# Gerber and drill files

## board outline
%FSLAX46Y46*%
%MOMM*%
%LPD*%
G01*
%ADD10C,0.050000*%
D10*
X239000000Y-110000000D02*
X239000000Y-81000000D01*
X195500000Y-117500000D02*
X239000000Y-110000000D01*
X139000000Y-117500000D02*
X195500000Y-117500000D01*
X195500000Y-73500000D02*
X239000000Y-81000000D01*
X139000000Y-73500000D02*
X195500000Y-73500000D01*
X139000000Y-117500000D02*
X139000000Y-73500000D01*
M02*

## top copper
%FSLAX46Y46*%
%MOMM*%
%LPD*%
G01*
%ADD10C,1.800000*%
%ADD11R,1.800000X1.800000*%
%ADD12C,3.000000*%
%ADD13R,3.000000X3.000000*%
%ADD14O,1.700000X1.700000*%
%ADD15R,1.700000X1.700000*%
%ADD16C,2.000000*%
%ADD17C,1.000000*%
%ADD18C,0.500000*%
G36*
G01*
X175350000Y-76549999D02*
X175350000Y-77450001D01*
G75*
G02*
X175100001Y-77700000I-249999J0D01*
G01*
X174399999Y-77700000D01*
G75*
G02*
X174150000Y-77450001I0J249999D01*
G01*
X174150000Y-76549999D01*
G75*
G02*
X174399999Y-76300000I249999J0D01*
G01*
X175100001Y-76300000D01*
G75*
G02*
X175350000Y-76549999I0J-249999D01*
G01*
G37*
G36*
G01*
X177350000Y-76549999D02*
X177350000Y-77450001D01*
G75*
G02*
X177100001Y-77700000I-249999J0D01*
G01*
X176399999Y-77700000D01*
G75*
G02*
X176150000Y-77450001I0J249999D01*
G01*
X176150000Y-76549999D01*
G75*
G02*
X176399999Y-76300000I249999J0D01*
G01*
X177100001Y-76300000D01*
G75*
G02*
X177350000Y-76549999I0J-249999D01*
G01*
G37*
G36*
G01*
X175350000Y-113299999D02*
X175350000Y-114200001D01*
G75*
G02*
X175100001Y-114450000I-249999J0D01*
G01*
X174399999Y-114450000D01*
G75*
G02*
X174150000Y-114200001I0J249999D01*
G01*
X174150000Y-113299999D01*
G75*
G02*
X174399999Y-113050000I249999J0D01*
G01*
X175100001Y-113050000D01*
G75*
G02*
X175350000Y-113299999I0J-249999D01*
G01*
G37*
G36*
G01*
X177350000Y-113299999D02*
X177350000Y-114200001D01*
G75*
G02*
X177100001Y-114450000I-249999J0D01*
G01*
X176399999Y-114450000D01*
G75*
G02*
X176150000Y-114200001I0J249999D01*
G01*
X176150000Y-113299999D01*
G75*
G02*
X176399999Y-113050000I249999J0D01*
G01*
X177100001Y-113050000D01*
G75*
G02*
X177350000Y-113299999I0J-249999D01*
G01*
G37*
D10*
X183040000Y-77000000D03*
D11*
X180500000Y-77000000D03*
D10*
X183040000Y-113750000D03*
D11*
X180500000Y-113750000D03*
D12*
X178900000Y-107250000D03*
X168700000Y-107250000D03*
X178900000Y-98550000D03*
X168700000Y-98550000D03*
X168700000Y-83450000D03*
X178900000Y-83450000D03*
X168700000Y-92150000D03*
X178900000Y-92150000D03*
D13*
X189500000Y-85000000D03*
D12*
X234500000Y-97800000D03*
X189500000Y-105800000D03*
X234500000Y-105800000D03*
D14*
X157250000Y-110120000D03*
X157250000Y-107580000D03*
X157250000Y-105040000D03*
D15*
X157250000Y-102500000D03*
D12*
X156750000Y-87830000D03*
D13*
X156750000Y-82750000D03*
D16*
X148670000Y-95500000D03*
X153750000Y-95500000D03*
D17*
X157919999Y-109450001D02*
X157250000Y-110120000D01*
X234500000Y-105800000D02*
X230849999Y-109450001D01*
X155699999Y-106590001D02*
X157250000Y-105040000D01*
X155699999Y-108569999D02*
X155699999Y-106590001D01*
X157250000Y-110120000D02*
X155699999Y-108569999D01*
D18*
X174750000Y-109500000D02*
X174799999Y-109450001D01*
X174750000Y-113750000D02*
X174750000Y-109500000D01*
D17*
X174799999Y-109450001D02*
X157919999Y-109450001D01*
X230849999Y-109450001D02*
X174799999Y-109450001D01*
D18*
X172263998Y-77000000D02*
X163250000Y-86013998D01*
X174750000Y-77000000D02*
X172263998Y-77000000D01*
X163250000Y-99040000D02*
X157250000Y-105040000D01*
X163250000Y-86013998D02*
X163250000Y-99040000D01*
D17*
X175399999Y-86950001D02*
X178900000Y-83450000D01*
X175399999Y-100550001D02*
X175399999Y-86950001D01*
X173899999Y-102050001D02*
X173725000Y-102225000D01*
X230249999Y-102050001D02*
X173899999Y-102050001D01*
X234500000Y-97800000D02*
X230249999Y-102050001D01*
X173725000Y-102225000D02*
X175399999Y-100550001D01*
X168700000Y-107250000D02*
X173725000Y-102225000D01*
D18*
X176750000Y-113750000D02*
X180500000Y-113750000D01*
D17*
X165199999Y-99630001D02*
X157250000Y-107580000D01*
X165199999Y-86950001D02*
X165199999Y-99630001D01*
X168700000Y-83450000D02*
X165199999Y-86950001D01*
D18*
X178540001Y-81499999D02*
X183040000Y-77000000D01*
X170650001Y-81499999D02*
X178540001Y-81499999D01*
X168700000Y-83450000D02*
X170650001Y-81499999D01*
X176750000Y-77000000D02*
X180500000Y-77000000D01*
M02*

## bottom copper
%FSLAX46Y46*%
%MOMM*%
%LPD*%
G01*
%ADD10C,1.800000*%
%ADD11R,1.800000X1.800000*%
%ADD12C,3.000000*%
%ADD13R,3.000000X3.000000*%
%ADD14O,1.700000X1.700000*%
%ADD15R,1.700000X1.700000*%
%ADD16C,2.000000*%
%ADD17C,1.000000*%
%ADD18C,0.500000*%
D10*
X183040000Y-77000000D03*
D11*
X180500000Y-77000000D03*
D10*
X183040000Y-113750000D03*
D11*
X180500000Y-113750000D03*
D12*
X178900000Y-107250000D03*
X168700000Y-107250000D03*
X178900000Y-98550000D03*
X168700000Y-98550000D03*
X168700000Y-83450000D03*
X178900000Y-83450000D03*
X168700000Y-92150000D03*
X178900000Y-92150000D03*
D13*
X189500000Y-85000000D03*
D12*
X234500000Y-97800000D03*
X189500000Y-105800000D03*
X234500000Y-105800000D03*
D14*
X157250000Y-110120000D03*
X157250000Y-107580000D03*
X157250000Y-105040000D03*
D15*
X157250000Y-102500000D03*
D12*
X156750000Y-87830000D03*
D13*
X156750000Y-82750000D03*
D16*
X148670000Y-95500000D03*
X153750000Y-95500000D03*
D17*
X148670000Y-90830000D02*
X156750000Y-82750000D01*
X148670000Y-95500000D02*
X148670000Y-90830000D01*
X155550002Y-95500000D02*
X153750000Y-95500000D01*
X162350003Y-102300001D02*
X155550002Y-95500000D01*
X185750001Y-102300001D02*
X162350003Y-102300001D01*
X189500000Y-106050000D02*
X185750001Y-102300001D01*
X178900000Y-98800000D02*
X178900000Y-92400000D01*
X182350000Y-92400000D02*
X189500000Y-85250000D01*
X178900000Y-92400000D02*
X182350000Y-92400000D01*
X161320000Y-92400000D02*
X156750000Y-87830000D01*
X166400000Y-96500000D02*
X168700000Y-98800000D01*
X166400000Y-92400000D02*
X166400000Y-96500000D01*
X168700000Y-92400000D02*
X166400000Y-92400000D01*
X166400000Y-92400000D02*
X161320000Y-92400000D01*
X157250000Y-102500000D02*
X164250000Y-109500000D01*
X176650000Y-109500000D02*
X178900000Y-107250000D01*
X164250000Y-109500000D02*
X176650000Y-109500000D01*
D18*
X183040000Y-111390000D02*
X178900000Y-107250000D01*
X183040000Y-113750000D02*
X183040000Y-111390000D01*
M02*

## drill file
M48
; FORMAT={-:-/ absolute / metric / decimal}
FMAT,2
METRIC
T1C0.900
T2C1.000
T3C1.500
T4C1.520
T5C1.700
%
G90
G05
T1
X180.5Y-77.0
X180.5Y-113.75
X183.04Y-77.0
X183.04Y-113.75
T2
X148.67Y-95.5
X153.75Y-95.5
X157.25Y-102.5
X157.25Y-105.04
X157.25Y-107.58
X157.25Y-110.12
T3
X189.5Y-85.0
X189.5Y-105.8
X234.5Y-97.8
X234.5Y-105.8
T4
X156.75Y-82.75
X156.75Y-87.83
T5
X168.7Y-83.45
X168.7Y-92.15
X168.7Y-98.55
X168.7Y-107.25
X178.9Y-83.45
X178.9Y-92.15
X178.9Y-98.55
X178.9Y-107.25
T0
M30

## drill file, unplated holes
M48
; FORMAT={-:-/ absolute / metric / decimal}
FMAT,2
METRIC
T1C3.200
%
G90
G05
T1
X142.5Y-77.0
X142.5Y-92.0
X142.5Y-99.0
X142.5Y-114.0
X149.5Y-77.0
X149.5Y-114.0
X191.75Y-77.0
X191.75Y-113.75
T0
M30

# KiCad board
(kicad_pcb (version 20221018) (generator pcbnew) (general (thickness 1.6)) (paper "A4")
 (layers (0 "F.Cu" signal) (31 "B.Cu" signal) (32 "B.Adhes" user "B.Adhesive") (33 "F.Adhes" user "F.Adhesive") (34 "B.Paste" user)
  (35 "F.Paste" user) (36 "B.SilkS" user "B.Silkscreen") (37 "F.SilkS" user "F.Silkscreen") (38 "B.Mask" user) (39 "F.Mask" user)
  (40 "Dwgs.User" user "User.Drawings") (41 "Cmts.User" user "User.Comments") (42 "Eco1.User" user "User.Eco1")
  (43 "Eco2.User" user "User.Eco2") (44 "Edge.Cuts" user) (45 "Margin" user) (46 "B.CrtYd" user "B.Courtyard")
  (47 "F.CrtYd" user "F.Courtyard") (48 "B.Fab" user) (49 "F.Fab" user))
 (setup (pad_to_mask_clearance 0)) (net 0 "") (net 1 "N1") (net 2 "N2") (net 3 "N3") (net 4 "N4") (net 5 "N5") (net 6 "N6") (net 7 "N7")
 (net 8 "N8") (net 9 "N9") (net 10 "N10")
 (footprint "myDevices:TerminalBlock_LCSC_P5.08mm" (layer "F.Cu") (at 156.75 82.75 -90)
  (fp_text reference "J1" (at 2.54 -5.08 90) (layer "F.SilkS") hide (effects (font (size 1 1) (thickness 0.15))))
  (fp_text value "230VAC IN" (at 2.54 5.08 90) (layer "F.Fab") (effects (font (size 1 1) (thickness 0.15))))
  (pad "1" thru_hole rect (at 0 0 270) (size 3 3) (drill 1.52) (layers "*.Cu" "*.Mask") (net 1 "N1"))
  (pad "2" thru_hole circle (at 5.08 0 270) (size 3 3) (drill 1.52) (layers "*.Cu" "*.Mask") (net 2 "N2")))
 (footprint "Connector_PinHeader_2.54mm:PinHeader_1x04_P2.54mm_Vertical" (layer "F.Cu") (at 157.25 102.5)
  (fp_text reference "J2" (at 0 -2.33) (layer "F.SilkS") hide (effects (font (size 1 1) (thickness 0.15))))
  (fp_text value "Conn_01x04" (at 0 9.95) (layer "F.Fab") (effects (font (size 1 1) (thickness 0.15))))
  (pad "1" thru_hole rect (at 0 0) (size 1.7 1.7) (drill 1) (layers "*.Cu" "*.Mask") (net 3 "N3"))
  (pad "2" thru_hole oval (at 0 2.54) (size 1.7 1.7) (drill 1) (layers "*.Cu" "*.Mask") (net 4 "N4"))
  (pad "3" thru_hole oval (at 0 5.08) (size 1.7 1.7) (drill 1) (layers "*.Cu" "*.Mask") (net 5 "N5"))
  (pad "4" thru_hole oval (at 0 7.62) (size 1.7 1.7) (drill 1) (layers "*.Cu" "*.Mask") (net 4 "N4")))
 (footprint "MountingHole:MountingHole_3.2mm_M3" (layer "F.Cu") (at 149.5 77)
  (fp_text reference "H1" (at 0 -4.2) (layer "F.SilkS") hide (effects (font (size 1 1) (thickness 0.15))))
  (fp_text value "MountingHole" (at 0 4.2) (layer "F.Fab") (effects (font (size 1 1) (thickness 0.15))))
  (pad "" np_thru_hole circle (at 0 0) (size 3.2 3.2) (drill 3.2) (layers "*.Cu" "*.Mask")))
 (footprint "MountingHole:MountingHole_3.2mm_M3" (layer "F.Cu") (at 149.5 114)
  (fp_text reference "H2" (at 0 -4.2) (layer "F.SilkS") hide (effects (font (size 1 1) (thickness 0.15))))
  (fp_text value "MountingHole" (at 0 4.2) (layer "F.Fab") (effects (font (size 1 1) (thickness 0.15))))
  (pad "" np_thru_hole circle (at 0 0) (size 3.2 3.2) (drill 3.2) (layers "*.Cu" "*.Mask")))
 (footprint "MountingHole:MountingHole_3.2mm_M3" (layer "F.Cu") (at 191.75 77)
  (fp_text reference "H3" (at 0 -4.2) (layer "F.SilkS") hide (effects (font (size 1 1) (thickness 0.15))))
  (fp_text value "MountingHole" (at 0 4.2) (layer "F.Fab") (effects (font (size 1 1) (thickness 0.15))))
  (pad "" np_thru_hole circle (at 0 0) (size 3.2 3.2) (drill 3.2) (layers "*.Cu" "*.Mask")))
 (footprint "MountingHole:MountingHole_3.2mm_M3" (layer "F.Cu") (at 191.75 113.75)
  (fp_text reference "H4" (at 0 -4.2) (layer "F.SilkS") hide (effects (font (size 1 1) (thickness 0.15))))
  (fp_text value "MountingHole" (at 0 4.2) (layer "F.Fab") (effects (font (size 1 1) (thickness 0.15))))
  (pad "" np_thru_hole circle (at 0 0) (size 3.2 3.2) (drill 3.2) (layers "*.Cu" "*.Mask")))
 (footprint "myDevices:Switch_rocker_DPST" (layer "F.Cu") (at 168.7 98.55)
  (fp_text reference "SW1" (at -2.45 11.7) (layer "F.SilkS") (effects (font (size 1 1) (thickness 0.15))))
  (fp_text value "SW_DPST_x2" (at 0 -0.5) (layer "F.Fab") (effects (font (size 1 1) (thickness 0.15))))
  (pad "1" thru_hole circle (at 0 0) (size 3 3) (drill 1.7) (layers "*.Cu" "*.Mask") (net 2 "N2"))
  (pad "2" thru_hole circle (at 10.2 0) (size 3 3) (drill 1.7) (layers "*.Cu" "*.Mask") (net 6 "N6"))
  (pad "3" thru_hole circle (at 0 8.7) (size 3 3) (drill 1.7) (layers "*.Cu" "*.Mask") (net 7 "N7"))
  (pad "4" thru_hole circle (at 10.2 8.7) (size 3 3) (drill 1.7) (layers "*.Cu" "*.Mask") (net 3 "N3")))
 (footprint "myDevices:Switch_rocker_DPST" (layer "F.Cu") (at 178.9 92.15 180)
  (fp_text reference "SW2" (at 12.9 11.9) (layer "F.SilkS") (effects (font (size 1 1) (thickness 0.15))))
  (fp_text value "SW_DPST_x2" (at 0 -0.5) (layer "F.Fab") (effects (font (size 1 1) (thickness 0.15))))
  (pad "1" thru_hole circle (at 0 0 180) (size 3 3) (drill 1.7) (layers "*.Cu" "*.Mask") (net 6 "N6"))
  (pad "2" thru_hole circle (at 10.2 0 180) (size 3 3) (drill 1.7) (layers "*.Cu" "*.Mask") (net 2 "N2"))
  (pad "3" thru_hole circle (at 0 8.7 180) (size 3 3) (drill 1.7) (layers "*.Cu" "*.Mask") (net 7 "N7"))
  (pad "4" thru_hole circle (at 10.2 8.7 180) (size 3 3) (drill 1.7) (layers "*.Cu" "*.Mask") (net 5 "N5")))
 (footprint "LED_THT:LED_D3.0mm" (layer "F.Cu") (at 180.5 113.75)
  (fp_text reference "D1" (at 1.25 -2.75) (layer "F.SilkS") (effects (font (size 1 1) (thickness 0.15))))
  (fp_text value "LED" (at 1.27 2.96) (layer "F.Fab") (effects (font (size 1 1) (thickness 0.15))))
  (pad "1" thru_hole rect (at 0 0) (size 1.8 1.8) (drill 0.9) (layers "*.Cu" "*.Mask") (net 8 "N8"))
  (pad "2" thru_hole circle (at 2.54 0) (size 1.8 1.8) (drill 0.9) (layers "*.Cu" "*.Mask") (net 3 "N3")))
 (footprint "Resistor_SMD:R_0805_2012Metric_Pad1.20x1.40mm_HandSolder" (layer "F.Cu") (at 175.75 113.75 180)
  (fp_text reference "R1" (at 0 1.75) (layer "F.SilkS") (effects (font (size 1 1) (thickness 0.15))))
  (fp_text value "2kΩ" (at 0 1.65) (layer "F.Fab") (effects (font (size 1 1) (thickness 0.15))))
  (pad "1" smd roundrect (at -1 0 180) (size 1.2 1.4) (layers "F.Cu" "F.Paste" "F.Mask") (roundrect_rratio 0.2083325) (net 8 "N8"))
  (pad "2" smd roundrect (at 1 0 180) (size 1.2 1.4) (layers "F.Cu" "F.Paste" "F.Mask") (roundrect_rratio 0.2083325) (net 4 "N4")))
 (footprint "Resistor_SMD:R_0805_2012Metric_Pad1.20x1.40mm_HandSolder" (layer "F.Cu") (at 175.75 77 180)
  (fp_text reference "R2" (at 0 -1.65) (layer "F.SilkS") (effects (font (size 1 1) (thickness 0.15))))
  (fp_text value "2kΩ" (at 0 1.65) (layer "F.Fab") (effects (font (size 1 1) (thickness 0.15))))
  (pad "1" smd roundrect (at -1 0 180) (size 1.2 1.4) (layers "F.Cu" "F.Paste" "F.Mask") (roundrect_rratio 0.2083325) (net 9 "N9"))
  (pad "2" smd roundrect (at 1 0 180) (size 1.2 1.4) (layers "F.Cu" "F.Paste" "F.Mask") (roundrect_rratio 0.2083325) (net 4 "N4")))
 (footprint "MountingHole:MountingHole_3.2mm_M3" (layer "F.Cu") (at 142.5 77)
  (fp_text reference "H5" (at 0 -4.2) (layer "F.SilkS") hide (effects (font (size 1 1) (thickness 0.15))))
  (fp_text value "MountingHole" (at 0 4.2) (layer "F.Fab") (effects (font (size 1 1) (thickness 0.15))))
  (pad "" np_thru_hole circle (at 0 0) (size 3.2 3.2) (drill 3.2) (layers "*.Cu" "*.Mask")))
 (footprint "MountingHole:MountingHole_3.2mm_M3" (layer "F.Cu") (at 142.5 92)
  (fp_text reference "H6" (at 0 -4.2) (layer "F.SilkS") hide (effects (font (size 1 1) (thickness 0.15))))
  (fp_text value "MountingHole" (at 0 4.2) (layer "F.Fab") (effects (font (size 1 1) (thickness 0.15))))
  (pad "" np_thru_hole circle (at 0 0) (size 3.2 3.2) (drill 3.2) (layers "*.Cu" "*.Mask")))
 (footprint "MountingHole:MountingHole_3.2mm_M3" (layer "F.Cu") (at 142.5 99)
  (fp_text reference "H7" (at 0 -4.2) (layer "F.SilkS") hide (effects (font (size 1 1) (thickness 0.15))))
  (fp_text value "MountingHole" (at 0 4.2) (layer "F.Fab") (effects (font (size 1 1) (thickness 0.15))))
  (pad "" np_thru_hole circle (at 0 0) (size 3.2 3.2) (drill 3.2) (layers "*.Cu" "*.Mask")))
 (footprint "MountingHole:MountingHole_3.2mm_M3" (layer "F.Cu") (at 142.5 114)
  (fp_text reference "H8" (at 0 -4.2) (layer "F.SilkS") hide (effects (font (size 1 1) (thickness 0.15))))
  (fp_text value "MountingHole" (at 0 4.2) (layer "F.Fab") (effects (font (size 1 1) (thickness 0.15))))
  (pad "" np_thru_hole circle (at 0 0) (size 3.2 3.2) (drill 3.2) (layers "*.Cu" "*.Mask")))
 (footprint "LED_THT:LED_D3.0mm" (layer "F.Cu") (at 180.5 77)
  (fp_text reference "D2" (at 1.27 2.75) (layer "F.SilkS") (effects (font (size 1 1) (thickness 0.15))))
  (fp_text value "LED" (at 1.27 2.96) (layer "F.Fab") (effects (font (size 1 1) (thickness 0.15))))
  (pad "1" thru_hole rect (at 0 0) (size 1.8 1.8) (drill 0.9) (layers "*.Cu" "*.Mask") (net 9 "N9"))
  (pad "2" thru_hole circle (at 2.54 0) (size 1.8 1.8) (drill 0.9) (layers "*.Cu" "*.Mask") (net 5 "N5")))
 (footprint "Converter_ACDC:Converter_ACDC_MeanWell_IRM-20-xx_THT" (layer "F.Cu") (at 189.5 85)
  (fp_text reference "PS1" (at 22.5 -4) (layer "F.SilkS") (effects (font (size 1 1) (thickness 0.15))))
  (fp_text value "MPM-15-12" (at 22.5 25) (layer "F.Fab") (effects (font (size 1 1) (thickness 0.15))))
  (pad "1" thru_hole rect (at 0 0) (size 3 3) (drill 1.5) (layers "*.Cu" "*.Mask") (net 6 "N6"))
  (pad "2" thru_hole circle (at 0 20.8) (size 3 3) (drill 1.5) (layers "*.Cu" "*.Mask") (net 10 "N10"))
  (pad "3" thru_hole circle (at 45 20.8) (size 3 3) (drill 1.5) (layers "*.Cu" "*.Mask") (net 4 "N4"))
  (pad "4" thru_hole circle (at 45 12.8) (size 3 3) (drill 1.5) (layers "*.Cu" "*.Mask") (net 7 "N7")))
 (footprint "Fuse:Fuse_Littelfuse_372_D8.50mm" (layer "F.Cu") (at 153.75 95.5 180)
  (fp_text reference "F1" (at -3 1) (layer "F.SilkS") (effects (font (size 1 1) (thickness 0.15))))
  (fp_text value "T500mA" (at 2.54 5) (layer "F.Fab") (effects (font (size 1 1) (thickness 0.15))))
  (pad "1" thru_hole circle (at 0 0 180) (size 2 2) (drill 1) (layers "*.Cu" "*.Mask") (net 10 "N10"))
  (pad "2" thru_hole circle (at 5.08 0 180) (size 2 2) (drill 1) (layers "*.Cu" "*.Mask") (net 1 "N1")))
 (gr_line (start 139 117.5) (end 139 73.5) (stroke (width 0.05) (type solid)) (layer "Edge.Cuts"))
 (gr_line (start 239 110) (end 239 81) (stroke (width 0.05) (type solid)) (layer "Edge.Cuts"))
 (gr_line (start 195.5 73.5) (end 239 81) (stroke (width 0.05) (type solid)) (layer "Edge.Cuts"))
 (gr_line (start 195.5 117.5) (end 239 110) (stroke (width 0.05) (type solid)) (layer "Edge.Cuts"))
 (gr_line (start 139 117.5) (end 195.5 117.5) (stroke (width 0.05) (type solid)) (layer "Edge.Cuts"))
 (gr_line (start 139 73.5) (end 195.5 73.5) (stroke (width 0.05) (type solid)) (layer "Edge.Cuts"))
 (segment (start 148.67 90.83) (end 156.75 82.75) (width 1) (layer "B.Cu") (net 1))
 (segment (start 148.67 95.5) (end 148.67 90.83) (width 1) (layer "B.Cu") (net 1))
 (segment (start 162.350003 102.300001) (end 155.550002 95.5) (width 1) (layer "B.Cu") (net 10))
 (segment (start 185.750001 102.300001) (end 162.350003 102.300001) (width 1) (layer "B.Cu") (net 10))
 (segment (start 155.550002 95.5) (end 153.75 95.5) (width 1) (layer "B.Cu") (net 10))
 (segment (start 189.5 106.05) (end 185.750001 102.300001) (width 1) (layer "B.Cu") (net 10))
 (segment (start 174.75 77) (end 172.263998 77) (width 0.5) (layer "F.Cu") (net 4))
 (segment (start 163.25 86.013998) (end 163.25 99.04) (width 0.5) (layer "F.Cu") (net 4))
 (segment (start 234.5 105.8) (end 230.849999 109.450001) (width 1) (layer "F.Cu") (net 4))
 (segment (start 163.25 99.04) (end 157.25 105.04) (width 0.5) (layer "F.Cu") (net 4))
 (segment (start 157.919999 109.450001) (end 157.25 110.12) (width 1) (layer "F.Cu") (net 4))
 (segment (start 230.849999 109.450001) (end 174.799999 109.450001) (width 1) (layer "F.Cu") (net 4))
 (segment (start 155.699999 106.590001) (end 157.25 105.04) (width 1) (layer "F.Cu") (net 4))
 (segment (start 172.263998 77) (end 163.25 86.013998) (width 0.5) (layer "F.Cu") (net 4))
 (segment (start 174.75 113.75) (end 174.75 109.5) (width 0.5) (layer "F.Cu") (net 4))
 (segment (start 157.25 110.12) (end 155.699999 108.569999) (width 1) (layer "F.Cu") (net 4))
 (segment (start 174.799999 109.450001) (end 157.919999 109.450001) (width 1) (layer "F.Cu") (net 4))
 (segment (start 174.75 109.5) (end 174.799999 109.450001) (width 0.5) (layer "F.Cu") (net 4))
 (segment (start 155.699999 108.569999) (end 155.699999 106.590001) (width 1) (layer "F.Cu") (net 4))
 (segment (start 182.35 92.4) (end 189.5 85.25) (width 1) (layer "B.Cu") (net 6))
 (segment (start 178.9 92.4) (end 182.35 92.4) (width 1) (layer "B.Cu") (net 6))
 (segment (start 178.9 98.8) (end 178.9 92.4) (width 1) (layer "B.Cu") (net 6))
 (segment (start 175.399999 100.550001) (end 175.399999 86.950001) (width 1) (layer "F.Cu") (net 7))
 (segment (start 175.399999 86.950001) (end 178.9 83.45) (width 1) (layer "F.Cu") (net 7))
 (segment (start 234.5 97.8) (end 230.249999 102.050001) (width 1) (layer "F.Cu") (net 7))
 (segment (start 173.899999 102.050001) (end 173.725 102.225) (width 1) (layer "F.Cu") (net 7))
 (segment (start 168.7 107.25) (end 173.725 102.225) (width 1) (layer "F.Cu") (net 7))
 (segment (start 173.725 102.225) (end 175.399999 100.550001) (width 1) (layer "F.Cu") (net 7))
 (segment (start 230.249999 102.050001) (end 173.899999 102.050001) (width 1) (layer "F.Cu") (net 7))
 (segment (start 161.32 92.4) (end 156.75 87.83) (width 1) (layer "B.Cu") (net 2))
 (segment (start 168.7 92.4) (end 166.4 92.4) (width 1) (layer "B.Cu") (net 2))
 (segment (start 166.4 92.4) (end 166.4 96.5) (width 1) (layer "B.Cu") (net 2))
 (segment (start 166.4 92.4) (end 161.32 92.4) (width 1) (layer "B.Cu") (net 2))
 (segment (start 166.4 96.5) (end 168.7 98.8) (width 1) (layer "B.Cu") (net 2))
 (segment (start 176.65 109.5) (end 178.9 107.25) (width 1) (layer "B.Cu") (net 3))
 (segment (start 183.04 113.75) (end 183.04 111.39) (width 0.5) (layer "B.Cu") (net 3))
 (segment (start 183.04 111.39) (end 178.9 107.25) (width 0.5) (layer "B.Cu") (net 3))
 (segment (start 164.25 109.5) (end 176.65 109.5) (width 1) (layer "B.Cu") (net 3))
 (segment (start 157.25 102.5) (end 164.25 109.5) (width 1) (layer "B.Cu") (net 3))
 (segment (start 176.75 113.75) (end 180.5 113.75) (width 0.5) (layer "F.Cu") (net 8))
 (segment (start 168.7 83.45) (end 170.650001 81.499999) (width 0.5) (layer "F.Cu") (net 5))
 (segment (start 168.7 83.45) (end 165.199999 86.950001) (width 1) (layer "F.Cu") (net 5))
 (segment (start 165.199999 86.950001) (end 165.199999 99.630001) (width 1) (layer "F.Cu") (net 5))
 (segment (start 170.650001 81.499999) (end 178.540001 81.499999) (width 0.5) (layer "F.Cu") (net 5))
 (segment (start 178.540001 81.499999) (end 183.04 77) (width 0.5) (layer "F.Cu") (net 5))
 (segment (start 165.199999 99.630001) (end 157.25 107.58) (width 1) (layer "F.Cu") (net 5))
 (segment (start 176.75 77) (end 180.5 77) (width 0.5) (layer "F.Cu") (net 9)))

